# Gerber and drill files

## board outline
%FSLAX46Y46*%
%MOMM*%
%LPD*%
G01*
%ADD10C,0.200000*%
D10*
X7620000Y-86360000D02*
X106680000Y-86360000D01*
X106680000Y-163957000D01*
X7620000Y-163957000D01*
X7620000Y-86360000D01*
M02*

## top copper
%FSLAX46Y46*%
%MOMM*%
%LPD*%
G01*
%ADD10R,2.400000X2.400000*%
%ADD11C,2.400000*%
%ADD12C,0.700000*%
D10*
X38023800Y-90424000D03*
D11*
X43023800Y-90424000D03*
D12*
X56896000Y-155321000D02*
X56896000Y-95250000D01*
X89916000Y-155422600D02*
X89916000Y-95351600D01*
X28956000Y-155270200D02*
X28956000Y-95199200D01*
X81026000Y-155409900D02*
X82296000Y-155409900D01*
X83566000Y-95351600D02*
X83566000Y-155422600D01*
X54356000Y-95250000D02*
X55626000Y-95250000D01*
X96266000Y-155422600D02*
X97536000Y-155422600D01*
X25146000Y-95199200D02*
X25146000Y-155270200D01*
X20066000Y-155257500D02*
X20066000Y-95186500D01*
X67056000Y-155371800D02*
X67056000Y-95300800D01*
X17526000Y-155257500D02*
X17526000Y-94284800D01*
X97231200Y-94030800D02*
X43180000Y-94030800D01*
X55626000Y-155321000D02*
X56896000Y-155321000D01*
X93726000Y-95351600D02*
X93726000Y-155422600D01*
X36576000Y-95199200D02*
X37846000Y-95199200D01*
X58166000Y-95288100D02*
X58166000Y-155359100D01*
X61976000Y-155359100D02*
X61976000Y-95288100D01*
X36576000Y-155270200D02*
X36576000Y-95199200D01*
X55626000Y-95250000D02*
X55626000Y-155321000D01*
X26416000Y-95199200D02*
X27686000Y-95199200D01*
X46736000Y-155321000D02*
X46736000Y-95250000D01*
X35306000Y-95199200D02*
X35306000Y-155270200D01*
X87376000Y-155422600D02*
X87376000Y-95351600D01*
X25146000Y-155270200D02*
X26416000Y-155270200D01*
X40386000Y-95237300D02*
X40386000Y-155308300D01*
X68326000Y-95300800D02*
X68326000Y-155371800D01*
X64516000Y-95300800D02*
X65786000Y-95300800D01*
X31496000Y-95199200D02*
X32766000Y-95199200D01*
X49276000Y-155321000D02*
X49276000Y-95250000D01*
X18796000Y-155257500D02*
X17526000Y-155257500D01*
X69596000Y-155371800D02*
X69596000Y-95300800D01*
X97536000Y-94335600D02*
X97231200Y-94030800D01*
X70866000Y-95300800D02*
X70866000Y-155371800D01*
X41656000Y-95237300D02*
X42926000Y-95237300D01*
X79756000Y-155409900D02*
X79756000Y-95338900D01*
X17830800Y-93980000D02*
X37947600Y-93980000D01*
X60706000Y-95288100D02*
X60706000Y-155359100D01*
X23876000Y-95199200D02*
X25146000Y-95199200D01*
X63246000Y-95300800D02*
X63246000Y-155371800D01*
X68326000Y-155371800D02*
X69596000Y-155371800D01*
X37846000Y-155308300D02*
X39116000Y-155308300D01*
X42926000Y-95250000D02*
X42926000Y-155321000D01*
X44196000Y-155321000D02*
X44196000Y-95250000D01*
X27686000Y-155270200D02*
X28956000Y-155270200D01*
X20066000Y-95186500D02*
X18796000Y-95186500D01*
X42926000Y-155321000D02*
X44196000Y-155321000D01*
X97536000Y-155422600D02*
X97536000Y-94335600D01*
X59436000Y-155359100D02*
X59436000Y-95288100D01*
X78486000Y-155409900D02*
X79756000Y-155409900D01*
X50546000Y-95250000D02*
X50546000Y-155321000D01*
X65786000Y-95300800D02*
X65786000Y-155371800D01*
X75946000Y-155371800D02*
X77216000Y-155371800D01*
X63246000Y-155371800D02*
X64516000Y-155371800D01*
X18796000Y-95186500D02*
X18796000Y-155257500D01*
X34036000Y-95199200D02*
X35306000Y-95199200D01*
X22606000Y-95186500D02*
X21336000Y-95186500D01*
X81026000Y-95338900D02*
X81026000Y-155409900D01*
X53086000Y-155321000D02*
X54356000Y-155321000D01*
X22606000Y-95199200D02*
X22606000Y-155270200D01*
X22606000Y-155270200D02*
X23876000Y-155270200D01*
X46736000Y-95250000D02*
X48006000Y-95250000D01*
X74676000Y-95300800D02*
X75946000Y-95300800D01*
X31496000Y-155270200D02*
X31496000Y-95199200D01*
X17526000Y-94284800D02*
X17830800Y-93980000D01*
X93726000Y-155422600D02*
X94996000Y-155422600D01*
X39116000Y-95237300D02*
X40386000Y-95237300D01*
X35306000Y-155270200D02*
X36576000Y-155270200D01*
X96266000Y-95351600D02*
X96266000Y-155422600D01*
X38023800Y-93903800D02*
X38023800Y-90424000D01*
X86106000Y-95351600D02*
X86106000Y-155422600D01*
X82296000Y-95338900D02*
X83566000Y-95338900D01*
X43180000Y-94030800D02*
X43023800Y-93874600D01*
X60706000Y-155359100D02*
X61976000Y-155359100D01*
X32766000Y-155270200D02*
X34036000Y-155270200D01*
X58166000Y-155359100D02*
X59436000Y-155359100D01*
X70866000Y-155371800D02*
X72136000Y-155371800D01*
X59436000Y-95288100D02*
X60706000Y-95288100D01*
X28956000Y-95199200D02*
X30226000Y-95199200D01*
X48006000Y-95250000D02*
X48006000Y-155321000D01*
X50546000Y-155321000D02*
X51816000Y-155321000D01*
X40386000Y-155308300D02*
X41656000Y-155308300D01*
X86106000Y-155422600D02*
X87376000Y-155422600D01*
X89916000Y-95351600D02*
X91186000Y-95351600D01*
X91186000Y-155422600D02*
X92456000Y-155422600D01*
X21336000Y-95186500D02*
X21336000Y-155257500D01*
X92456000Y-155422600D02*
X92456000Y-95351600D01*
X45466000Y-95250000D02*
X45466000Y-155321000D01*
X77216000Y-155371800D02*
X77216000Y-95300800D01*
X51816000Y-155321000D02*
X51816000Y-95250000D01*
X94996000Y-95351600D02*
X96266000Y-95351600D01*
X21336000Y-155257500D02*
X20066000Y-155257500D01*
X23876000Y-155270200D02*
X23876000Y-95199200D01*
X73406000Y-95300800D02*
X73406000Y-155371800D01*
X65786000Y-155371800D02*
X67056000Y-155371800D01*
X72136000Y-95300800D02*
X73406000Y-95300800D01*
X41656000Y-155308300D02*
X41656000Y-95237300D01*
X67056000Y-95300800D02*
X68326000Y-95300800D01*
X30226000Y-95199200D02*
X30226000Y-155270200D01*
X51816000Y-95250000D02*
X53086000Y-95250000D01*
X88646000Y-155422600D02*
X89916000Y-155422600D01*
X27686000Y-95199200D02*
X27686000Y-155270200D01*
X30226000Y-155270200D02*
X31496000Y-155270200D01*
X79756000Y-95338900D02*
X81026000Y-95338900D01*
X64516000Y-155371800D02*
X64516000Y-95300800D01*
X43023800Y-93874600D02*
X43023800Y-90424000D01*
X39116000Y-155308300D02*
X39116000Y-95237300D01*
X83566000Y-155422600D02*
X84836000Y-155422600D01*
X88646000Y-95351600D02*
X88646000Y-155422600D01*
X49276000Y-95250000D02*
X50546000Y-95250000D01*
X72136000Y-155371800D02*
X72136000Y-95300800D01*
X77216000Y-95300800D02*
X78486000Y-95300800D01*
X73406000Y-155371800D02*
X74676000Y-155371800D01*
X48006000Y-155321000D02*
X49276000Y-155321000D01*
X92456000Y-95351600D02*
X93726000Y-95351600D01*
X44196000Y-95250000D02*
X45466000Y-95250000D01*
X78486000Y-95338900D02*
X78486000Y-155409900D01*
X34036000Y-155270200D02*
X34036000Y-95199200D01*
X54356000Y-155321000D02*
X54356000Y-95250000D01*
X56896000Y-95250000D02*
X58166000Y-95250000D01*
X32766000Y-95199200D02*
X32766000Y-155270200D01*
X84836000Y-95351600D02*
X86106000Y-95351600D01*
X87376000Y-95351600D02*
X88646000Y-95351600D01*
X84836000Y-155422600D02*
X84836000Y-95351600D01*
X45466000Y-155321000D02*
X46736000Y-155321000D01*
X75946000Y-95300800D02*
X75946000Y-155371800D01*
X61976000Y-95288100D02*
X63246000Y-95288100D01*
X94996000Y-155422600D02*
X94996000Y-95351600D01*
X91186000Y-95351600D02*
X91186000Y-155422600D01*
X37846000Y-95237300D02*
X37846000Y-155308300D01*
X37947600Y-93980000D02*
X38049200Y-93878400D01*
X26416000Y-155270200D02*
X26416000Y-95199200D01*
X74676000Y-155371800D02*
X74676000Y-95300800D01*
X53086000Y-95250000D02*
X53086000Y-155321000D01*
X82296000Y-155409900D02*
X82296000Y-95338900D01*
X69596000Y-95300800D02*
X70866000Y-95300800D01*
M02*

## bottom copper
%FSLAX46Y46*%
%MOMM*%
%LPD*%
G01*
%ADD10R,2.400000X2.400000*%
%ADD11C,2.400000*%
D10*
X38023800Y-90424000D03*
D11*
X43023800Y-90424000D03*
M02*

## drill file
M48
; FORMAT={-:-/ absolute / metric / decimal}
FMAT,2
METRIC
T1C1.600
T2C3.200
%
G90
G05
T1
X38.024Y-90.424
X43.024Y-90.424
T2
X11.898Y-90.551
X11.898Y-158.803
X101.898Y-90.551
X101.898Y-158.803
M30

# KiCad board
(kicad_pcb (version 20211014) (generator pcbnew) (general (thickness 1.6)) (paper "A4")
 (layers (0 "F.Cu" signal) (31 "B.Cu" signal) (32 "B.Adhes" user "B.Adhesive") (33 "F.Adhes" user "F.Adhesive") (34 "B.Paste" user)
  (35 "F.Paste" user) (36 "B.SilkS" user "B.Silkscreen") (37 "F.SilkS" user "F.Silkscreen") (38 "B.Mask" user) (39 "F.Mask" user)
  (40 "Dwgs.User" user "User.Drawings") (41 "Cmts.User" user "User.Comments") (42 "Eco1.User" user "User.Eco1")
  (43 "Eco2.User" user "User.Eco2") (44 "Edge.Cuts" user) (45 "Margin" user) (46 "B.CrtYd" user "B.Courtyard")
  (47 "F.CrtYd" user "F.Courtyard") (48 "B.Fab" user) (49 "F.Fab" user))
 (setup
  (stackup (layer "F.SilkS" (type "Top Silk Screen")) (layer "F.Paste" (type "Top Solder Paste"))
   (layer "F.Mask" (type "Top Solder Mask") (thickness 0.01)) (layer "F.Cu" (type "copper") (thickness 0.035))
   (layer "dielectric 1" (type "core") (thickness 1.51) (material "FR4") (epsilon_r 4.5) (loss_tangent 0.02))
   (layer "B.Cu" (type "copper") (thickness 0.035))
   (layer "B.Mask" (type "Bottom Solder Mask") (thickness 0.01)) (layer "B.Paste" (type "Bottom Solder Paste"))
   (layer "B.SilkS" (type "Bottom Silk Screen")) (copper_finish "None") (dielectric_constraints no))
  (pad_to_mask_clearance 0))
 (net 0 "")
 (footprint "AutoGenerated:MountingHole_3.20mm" (layer "F.Cu") (at 91.898 142.803)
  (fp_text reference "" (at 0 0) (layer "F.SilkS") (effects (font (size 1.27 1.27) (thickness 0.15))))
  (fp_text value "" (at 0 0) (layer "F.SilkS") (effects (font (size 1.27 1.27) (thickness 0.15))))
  (pad "" np_thru_hole circle (at 10 16) (size 3.2 3.2) (drill 3.2) (layers F&B.Cu *.Mask)))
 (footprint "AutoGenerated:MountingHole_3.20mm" (layer "F.Cu") (at 11.898 90.551)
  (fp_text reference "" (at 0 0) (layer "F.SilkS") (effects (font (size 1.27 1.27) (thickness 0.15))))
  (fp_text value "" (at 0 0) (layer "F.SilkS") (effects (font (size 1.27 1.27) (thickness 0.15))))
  (pad "" np_thru_hole circle locked (at 0 0) (size 3.2 3.2) (drill 3.2) (layers *.Cu *.Mask)))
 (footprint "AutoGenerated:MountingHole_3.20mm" (layer "F.Cu") (at 91.898 90.551)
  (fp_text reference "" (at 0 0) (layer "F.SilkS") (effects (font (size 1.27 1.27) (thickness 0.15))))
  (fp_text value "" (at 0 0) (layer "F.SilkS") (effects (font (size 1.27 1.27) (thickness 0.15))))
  (pad "" np_thru_hole circle (at 10 0) (size 3.2 3.2) (drill 3.2) (layers F&B.Cu *.Mask)))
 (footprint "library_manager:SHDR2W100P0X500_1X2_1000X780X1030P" (layer "F.Cu") (at 38.0238 90.424)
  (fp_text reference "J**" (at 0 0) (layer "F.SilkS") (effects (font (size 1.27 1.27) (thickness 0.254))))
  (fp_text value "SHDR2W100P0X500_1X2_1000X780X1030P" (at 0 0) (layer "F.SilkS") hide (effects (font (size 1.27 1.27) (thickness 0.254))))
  (pad "1" thru_hole rect locked (at 0 0) (size 2.4 2.4) (drill 1.6) (layers *.Cu *.Mask))
  (pad "2" thru_hole circle locked (at 5 0) (size 2.4 2.4) (drill 1.6) (layers *.Cu *.Mask)))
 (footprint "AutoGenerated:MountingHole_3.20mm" (layer "F.Cu") (at 11.898 142.803)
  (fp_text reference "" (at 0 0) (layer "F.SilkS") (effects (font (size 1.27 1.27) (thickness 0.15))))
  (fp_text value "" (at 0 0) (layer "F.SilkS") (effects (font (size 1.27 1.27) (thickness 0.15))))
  (pad "" np_thru_hole circle (at 0 16) (size 3.2 3.2) (drill 3.2) (layers F&B.Cu *.Mask)))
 (gr_rect (start 7.62 86.36) (end 106.68 163.957) (layer "Edge.Cuts") (width 0.2) (fill none))
 (segment (start 56.896 155.321) (end 56.896 95.25) (width 0.7) (layer "F.Cu") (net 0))
 (segment (start 89.916 155.4226) (end 89.916 95.3516) (width 0.7) (layer "F.Cu") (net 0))
 (segment (start 28.956 155.2702) (end 28.956 95.1992) (width 0.7) (layer "F.Cu") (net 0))
 (segment (start 81.026 155.4099) (end 82.296 155.4099) (width 0.7) (layer "F.Cu") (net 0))
 (segment (start 83.566 95.3516) (end 83.566 155.4226) (width 0.7) (layer "F.Cu") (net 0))
 (segment (start 54.356 95.25) (end 55.626 95.25) (width 0.7) (layer "F.Cu") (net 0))
 (segment (start 96.266 155.4226) (end 97.536 155.4226) (width 0.7) (layer "F.Cu") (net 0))
 (segment (start 25.146 95.1992) (end 25.146 155.2702) (width 0.7) (layer "F.Cu") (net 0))
 (segment (start 20.066 155.2575) (end 20.066 95.1865) (width 0.7) (layer "F.Cu") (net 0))
 (segment (start 67.056 155.3718) (end 67.056 95.3008) (width 0.7) (layer "F.Cu") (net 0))
 (segment (start 17.526 155.2575) (end 17.526 94.2848) (width 0.7) (layer "F.Cu") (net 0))
 (segment (start 97.2312 94.0308) (end 43.18 94.0308) (width 0.7) (layer "F.Cu") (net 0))
 (segment (start 55.626 155.321) (end 56.896 155.321) (width 0.7) (layer "F.Cu") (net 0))
 (segment (start 93.726 95.3516) (end 93.726 155.4226) (width 0.7) (layer "F.Cu") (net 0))
 (segment (start 36.576 95.1992) (end 37.846 95.1992) (width 0.7) (layer "F.Cu") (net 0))
 (segment (start 58.166 95.2881) (end 58.166 155.3591) (width 0.7) (layer "F.Cu") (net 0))
 (segment (start 61.976 155.3591) (end 61.976 95.2881) (width 0.7) (layer "F.Cu") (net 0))
 (segment (start 36.576 155.2702) (end 36.576 95.1992) (width 0.7) (layer "F.Cu") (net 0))
 (segment (start 55.626 95.25) (end 55.626 155.321) (width 0.7) (layer "F.Cu") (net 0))
 (segment (start 26.416 95.1992) (end 27.686 95.1992) (width 0.7) (layer "F.Cu") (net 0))
 (segment (start 46.736 155.321) (end 46.736 95.25) (width 0.7) (layer "F.Cu") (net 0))
 (segment (start 35.306 95.1992) (end 35.306 155.2702) (width 0.7) (layer "F.Cu") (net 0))
 (segment (start 87.376 155.4226) (end 87.376 95.3516) (width 0.7) (layer "F.Cu") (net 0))
 (segment (start 25.146 155.2702) (end 26.416 155.2702) (width 0.7) (layer "F.Cu") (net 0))
 (segment (start 40.386 95.2373) (end 40.386 155.3083) (width 0.7) (layer "F.Cu") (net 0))
 (segment (start 68.326 95.3008) (end 68.326 155.3718) (width 0.7) (layer "F.Cu") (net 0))
 (segment (start 64.516 95.3008) (end 65.786 95.3008) (width 0.7) (layer "F.Cu") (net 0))
 (segment (start 31.496 95.1992) (end 32.766 95.1992) (width 0.7) (layer "F.Cu") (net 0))
 (segment (start 49.276 155.321) (end 49.276 95.25) (width 0.7) (layer "F.Cu") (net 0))
 (segment (start 18.796 155.2575) (end 17.526 155.2575) (width 0.7) (layer "F.Cu") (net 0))
 (segment (start 69.596 155.3718) (end 69.596 95.3008) (width 0.7) (layer "F.Cu") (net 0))
 (segment (start 97.536 94.3356) (end 97.2312 94.0308) (width 0.7) (layer "F.Cu") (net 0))
 (segment (start 70.866 95.3008) (end 70.866 155.3718) (width 0.7) (layer "F.Cu") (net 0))
 (segment (start 41.656 95.2373) (end 42.926 95.2373) (width 0.7) (layer "F.Cu") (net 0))
 (segment (start 79.756 155.4099) (end 79.756 95.3389) (width 0.7) (layer "F.Cu") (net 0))
 (segment (start 17.8308 93.98) (end 37.9476 93.98) (width 0.7) (layer "F.Cu") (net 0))
 (segment (start 60.706 95.2881) (end 60.706 155.3591) (width 0.7) (layer "F.Cu") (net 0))
 (segment (start 23.876 95.1992) (end 25.146 95.1992) (width 0.7) (layer "F.Cu") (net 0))
 (segment (start 63.246 95.3008) (end 63.246 155.3718) (width 0.7) (layer "F.Cu") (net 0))
 (segment (start 68.326 155.3718) (end 69.596 155.3718) (width 0.7) (layer "F.Cu") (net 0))
 (segment (start 37.846 155.3083) (end 39.116 155.3083) (width 0.7) (layer "F.Cu") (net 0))
 (segment (start 42.926 95.25) (end 42.926 155.321) (width 0.7) (layer "F.Cu") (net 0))
 (segment (start 44.196 155.321) (end 44.196 95.25) (width 0.7) (layer "F.Cu") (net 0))
 (segment (start 27.686 155.2702) (end 28.956 155.2702) (width 0.7) (layer "F.Cu") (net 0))
 (segment (start 20.066 95.1865) (end 18.796 95.1865) (width 0.7) (layer "F.Cu") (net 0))
 (segment (start 42.926 155.321) (end 44.196 155.321) (width 0.7) (layer "F.Cu") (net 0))
 (segment (start 97.536 155.4226) (end 97.536 94.3356) (width 0.7) (layer "F.Cu") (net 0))
 (segment (start 59.436 155.3591) (end 59.436 95.2881) (width 0.7) (layer "F.Cu") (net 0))
 (segment (start 78.486 155.4099) (end 79.756 155.4099) (width 0.7) (layer "F.Cu") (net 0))
 (segment (start 50.546 95.25) (end 50.546 155.321) (width 0.7) (layer "F.Cu") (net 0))
 (segment (start 65.786 95.3008) (end 65.786 155.3718) (width 0.7) (layer "F.Cu") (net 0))
 (segment (start 75.946 155.3718) (end 77.216 155.3718) (width 0.7) (layer "F.Cu") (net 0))
 (segment (start 63.246 155.3718) (end 64.516 155.3718) (width 0.7) (layer "F.Cu") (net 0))
 (segment (start 18.796 95.1865) (end 18.796 155.2575) (width 0.7) (layer "F.Cu") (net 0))
 (segment (start 34.036 95.1992) (end 35.306 95.1992) (width 0.7) (layer "F.Cu") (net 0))
 (segment (start 22.606 95.1865) (end 21.336 95.1865) (width 0.7) (layer "F.Cu") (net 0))
 (segment (start 81.026 95.3389) (end 81.026 155.4099) (width 0.7) (layer "F.Cu") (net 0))
 (segment (start 53.086 155.321) (end 54.356 155.321) (width 0.7) (layer "F.Cu") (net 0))
 (segment (start 22.606 95.1992) (end 22.606 155.2702) (width 0.7) (layer "F.Cu") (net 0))
 (segment (start 22.606 155.2702) (end 23.876 155.2702) (width 0.7) (layer "F.Cu") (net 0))
 (segment (start 46.736 95.25) (end 48.006 95.25) (width 0.7) (layer "F.Cu") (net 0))
 (segment (start 74.676 95.3008) (end 75.946 95.3008) (width 0.7) (layer "F.Cu") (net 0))
 (segment (start 31.496 155.2702) (end 31.496 95.1992) (width 0.7) (layer "F.Cu") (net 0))
 (segment (start 17.526 94.2848) (end 17.8308 93.98) (width 0.7) (layer "F.Cu") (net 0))
 (segment (start 93.726 155.4226) (end 94.996 155.4226) (width 0.7) (layer "F.Cu") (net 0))
 (segment (start 39.116 95.2373) (end 40.386 95.2373) (width 0.7) (layer "F.Cu") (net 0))
 (segment (start 35.306 155.2702) (end 36.576 155.2702) (width 0.7) (layer "F.Cu") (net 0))
 (segment (start 96.266 95.3516) (end 96.266 155.4226) (width 0.7) (layer "F.Cu") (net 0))
 (segment (start 38.0238 93.9038) (end 38.0238 90.424) (width 0.7) (layer "F.Cu") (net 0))
 (segment (start 86.106 95.3516) (end 86.106 155.4226) (width 0.7) (layer "F.Cu") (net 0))
 (segment (start 82.296 95.3389) (end 83.566 95.3389) (width 0.7) (layer "F.Cu") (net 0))
 (segment (start 43.18 94.0308) (end 43.0238 93.8746) (width 0.7) (layer "F.Cu") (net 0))
 (segment (start 60.706 155.3591) (end 61.976 155.3591) (width 0.7) (layer "F.Cu") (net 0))
 (segment (start 32.766 155.2702) (end 34.036 155.2702) (width 0.7) (layer "F.Cu") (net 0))
 (segment (start 58.166 155.3591) (end 59.436 155.3591) (width 0.7) (layer "F.Cu") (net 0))
 (segment (start 70.866 155.3718) (end 72.136 155.3718) (width 0.7) (layer "F.Cu") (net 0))
 (segment (start 59.436 95.2881) (end 60.706 95.2881) (width 0.7) (layer "F.Cu") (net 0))
 (segment (start 28.956 95.1992) (end 30.226 95.1992) (width 0.7) (layer "F.Cu") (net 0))
 (segment (start 48.006 95.25) (end 48.006 155.321) (width 0.7) (layer "F.Cu") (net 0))
 (segment (start 50.546 155.321) (end 51.816 155.321) (width 0.7) (layer "F.Cu") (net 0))
 (segment (start 40.386 155.3083) (end 41.656 155.3083) (width 0.7) (layer "F.Cu") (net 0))
 (segment (start 86.106 155.4226) (end 87.376 155.4226) (width 0.7) (layer "F.Cu") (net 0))
 (segment (start 89.916 95.3516) (end 91.186 95.3516) (width 0.7) (layer "F.Cu") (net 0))
 (segment (start 91.186 155.4226) (end 92.456 155.4226) (width 0.7) (layer "F.Cu") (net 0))
 (segment (start 21.336 95.1865) (end 21.336 155.2575) (width 0.7) (layer "F.Cu") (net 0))
 (segment (start 92.456 155.4226) (end 92.456 95.3516) (width 0.7) (layer "F.Cu") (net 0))
 (segment (start 45.466 95.25) (end 45.466 155.321) (width 0.7) (layer "F.Cu") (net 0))
 (segment (start 77.216 155.3718) (end 77.216 95.3008) (width 0.7) (layer "F.Cu") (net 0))
 (segment (start 51.816 155.321) (end 51.816 95.25) (width 0.7) (layer "F.Cu") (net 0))
 (segment (start 94.996 95.3516) (end 96.266 95.3516) (width 0.7) (layer "F.Cu") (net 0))
 (segment (start 21.336 155.2575) (end 20.066 155.2575) (width 0.7) (layer "F.Cu") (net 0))
 (segment (start 23.876 155.2702) (end 23.876 95.1992) (width 0.7) (layer "F.Cu") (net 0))
 (segment (start 73.406 95.3008) (end 73.406 155.3718) (width 0.7) (layer "F.Cu") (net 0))
 (segment (start 65.786 155.3718) (end 67.056 155.3718) (width 0.7) (layer "F.Cu") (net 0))
 (segment (start 72.136 95.3008) (end 73.406 95.3008) (width 0.7) (layer "F.Cu") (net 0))
 (segment (start 41.656 155.3083) (end 41.656 95.2373) (width 0.7) (layer "F.Cu") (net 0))
 (segment (start 67.056 95.3008) (end 68.326 95.3008) (width 0.7) (layer "F.Cu") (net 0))
 (segment (start 30.226 95.1992) (end 30.226 155.2702) (width 0.7) (layer "F.Cu") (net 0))
 (segment (start 51.816 95.25) (end 53.086 95.25) (width 0.7) (layer "F.Cu") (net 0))
 (segment (start 88.646 155.4226) (end 89.916 155.4226) (width 0.7) (layer "F.Cu") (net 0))
 (segment (start 27.686 95.1992) (end 27.686 155.2702) (width 0.7) (layer "F.Cu") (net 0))
 (segment (start 30.226 155.2702) (end 31.496 155.2702) (width 0.7) (layer "F.Cu") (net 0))
 (segment (start 79.756 95.3389) (end 81.026 95.3389) (width 0.7) (layer "F.Cu") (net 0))
 (segment (start 64.516 155.3718) (end 64.516 95.3008) (width 0.7) (layer "F.Cu") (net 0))
 (segment (start 43.0238 93.8746) (end 43.0238 90.424) (width 0.7) (layer "F.Cu") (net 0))
 (segment (start 39.116 155.3083) (end 39.116 95.2373) (width 0.7) (layer "F.Cu") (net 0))
 (segment (start 83.566 155.4226) (end 84.836 155.4226) (width 0.7) (layer "F.Cu") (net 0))
 (segment (start 88.646 95.3516) (end 88.646 155.4226) (width 0.7) (layer "F.Cu") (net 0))
 (segment (start 49.276 95.25) (end 50.546 95.25) (width 0.7) (layer "F.Cu") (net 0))
 (segment (start 72.136 155.3718) (end 72.136 95.3008) (width 0.7) (layer "F.Cu") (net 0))
 (segment (start 77.216 95.3008) (end 78.486 95.3008) (width 0.7) (layer "F.Cu") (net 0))
 (segment (start 73.406 155.3718) (end 74.676 155.3718) (width 0.7) (layer "F.Cu") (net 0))
 (segment (start 48.006 155.321) (end 49.276 155.321) (width 0.7) (layer "F.Cu") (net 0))
 (segment (start 92.456 95.3516) (end 93.726 95.3516) (width 0.7) (layer "F.Cu") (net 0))
 (segment (start 44.196 95.25) (end 45.466 95.25) (width 0.7) (layer "F.Cu") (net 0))
 (segment (start 78.486 95.3389) (end 78.486 155.4099) (width 0.7) (layer "F.Cu") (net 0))
 (segment (start 34.036 155.2702) (end 34.036 95.1992) (width 0.7) (layer "F.Cu") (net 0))
 (segment (start 54.356 155.321) (end 54.356 95.25) (width 0.7) (layer "F.Cu") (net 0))
 (segment (start 56.896 95.25) (end 58.166 95.25) (width 0.7) (layer "F.Cu") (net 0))
 (segment (start 32.766 95.1992) (end 32.766 155.2702) (width 0.7) (layer "F.Cu") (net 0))
 (segment (start 84.836 95.3516) (end 86.106 95.3516) (width 0.7) (layer "F.Cu") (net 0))
 (segment (start 87.376 95.3516) (end 88.646 95.3516) (width 0.7) (layer "F.Cu") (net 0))
 (segment (start 84.836 155.4226) (end 84.836 95.3516) (width 0.7) (layer "F.Cu") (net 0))
 (segment (start 45.466 155.321) (end 46.736 155.321) (width 0.7) (layer "F.Cu") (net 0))
 (segment (start 75.946 95.3008) (end 75.946 155.3718) (width 0.7) (layer "F.Cu") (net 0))
 (segment (start 61.976 95.2881) (end 63.246 95.2881) (width 0.7) (layer "F.Cu") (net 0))
 (segment (start 94.996 155.4226) (end 94.996 95.3516) (width 0.7) (layer "F.Cu") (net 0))
 (segment (start 91.186 95.3516) (end 91.186 155.4226) (width 0.7) (layer "F.Cu") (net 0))
 (segment (start 37.846 95.2373) (end 37.846 155.3083) (width 0.7) (layer "F.Cu") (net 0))
 (segment (start 37.9476 93.98) (end 38.0492 93.8784) (width 0.7) (layer "F.Cu") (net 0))
 (segment (start 26.416 155.2702) (end 26.416 95.1992) (width 0.7) (layer "F.Cu") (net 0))
 (segment (start 74.676 155.3718) (end 74.676 95.3008) (width 0.7) (layer "F.Cu") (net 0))
 (segment (start 53.086 95.25) (end 53.086 155.321) (width 0.7) (layer "F.Cu") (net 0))
 (segment (start 82.296 155.4099) (end 82.296 95.3389) (width 0.7) (layer "F.Cu") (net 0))
 (segment (start 69.596 95.3008) (end 70.866 95.3008) (width 0.7) (layer "F.Cu") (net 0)))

